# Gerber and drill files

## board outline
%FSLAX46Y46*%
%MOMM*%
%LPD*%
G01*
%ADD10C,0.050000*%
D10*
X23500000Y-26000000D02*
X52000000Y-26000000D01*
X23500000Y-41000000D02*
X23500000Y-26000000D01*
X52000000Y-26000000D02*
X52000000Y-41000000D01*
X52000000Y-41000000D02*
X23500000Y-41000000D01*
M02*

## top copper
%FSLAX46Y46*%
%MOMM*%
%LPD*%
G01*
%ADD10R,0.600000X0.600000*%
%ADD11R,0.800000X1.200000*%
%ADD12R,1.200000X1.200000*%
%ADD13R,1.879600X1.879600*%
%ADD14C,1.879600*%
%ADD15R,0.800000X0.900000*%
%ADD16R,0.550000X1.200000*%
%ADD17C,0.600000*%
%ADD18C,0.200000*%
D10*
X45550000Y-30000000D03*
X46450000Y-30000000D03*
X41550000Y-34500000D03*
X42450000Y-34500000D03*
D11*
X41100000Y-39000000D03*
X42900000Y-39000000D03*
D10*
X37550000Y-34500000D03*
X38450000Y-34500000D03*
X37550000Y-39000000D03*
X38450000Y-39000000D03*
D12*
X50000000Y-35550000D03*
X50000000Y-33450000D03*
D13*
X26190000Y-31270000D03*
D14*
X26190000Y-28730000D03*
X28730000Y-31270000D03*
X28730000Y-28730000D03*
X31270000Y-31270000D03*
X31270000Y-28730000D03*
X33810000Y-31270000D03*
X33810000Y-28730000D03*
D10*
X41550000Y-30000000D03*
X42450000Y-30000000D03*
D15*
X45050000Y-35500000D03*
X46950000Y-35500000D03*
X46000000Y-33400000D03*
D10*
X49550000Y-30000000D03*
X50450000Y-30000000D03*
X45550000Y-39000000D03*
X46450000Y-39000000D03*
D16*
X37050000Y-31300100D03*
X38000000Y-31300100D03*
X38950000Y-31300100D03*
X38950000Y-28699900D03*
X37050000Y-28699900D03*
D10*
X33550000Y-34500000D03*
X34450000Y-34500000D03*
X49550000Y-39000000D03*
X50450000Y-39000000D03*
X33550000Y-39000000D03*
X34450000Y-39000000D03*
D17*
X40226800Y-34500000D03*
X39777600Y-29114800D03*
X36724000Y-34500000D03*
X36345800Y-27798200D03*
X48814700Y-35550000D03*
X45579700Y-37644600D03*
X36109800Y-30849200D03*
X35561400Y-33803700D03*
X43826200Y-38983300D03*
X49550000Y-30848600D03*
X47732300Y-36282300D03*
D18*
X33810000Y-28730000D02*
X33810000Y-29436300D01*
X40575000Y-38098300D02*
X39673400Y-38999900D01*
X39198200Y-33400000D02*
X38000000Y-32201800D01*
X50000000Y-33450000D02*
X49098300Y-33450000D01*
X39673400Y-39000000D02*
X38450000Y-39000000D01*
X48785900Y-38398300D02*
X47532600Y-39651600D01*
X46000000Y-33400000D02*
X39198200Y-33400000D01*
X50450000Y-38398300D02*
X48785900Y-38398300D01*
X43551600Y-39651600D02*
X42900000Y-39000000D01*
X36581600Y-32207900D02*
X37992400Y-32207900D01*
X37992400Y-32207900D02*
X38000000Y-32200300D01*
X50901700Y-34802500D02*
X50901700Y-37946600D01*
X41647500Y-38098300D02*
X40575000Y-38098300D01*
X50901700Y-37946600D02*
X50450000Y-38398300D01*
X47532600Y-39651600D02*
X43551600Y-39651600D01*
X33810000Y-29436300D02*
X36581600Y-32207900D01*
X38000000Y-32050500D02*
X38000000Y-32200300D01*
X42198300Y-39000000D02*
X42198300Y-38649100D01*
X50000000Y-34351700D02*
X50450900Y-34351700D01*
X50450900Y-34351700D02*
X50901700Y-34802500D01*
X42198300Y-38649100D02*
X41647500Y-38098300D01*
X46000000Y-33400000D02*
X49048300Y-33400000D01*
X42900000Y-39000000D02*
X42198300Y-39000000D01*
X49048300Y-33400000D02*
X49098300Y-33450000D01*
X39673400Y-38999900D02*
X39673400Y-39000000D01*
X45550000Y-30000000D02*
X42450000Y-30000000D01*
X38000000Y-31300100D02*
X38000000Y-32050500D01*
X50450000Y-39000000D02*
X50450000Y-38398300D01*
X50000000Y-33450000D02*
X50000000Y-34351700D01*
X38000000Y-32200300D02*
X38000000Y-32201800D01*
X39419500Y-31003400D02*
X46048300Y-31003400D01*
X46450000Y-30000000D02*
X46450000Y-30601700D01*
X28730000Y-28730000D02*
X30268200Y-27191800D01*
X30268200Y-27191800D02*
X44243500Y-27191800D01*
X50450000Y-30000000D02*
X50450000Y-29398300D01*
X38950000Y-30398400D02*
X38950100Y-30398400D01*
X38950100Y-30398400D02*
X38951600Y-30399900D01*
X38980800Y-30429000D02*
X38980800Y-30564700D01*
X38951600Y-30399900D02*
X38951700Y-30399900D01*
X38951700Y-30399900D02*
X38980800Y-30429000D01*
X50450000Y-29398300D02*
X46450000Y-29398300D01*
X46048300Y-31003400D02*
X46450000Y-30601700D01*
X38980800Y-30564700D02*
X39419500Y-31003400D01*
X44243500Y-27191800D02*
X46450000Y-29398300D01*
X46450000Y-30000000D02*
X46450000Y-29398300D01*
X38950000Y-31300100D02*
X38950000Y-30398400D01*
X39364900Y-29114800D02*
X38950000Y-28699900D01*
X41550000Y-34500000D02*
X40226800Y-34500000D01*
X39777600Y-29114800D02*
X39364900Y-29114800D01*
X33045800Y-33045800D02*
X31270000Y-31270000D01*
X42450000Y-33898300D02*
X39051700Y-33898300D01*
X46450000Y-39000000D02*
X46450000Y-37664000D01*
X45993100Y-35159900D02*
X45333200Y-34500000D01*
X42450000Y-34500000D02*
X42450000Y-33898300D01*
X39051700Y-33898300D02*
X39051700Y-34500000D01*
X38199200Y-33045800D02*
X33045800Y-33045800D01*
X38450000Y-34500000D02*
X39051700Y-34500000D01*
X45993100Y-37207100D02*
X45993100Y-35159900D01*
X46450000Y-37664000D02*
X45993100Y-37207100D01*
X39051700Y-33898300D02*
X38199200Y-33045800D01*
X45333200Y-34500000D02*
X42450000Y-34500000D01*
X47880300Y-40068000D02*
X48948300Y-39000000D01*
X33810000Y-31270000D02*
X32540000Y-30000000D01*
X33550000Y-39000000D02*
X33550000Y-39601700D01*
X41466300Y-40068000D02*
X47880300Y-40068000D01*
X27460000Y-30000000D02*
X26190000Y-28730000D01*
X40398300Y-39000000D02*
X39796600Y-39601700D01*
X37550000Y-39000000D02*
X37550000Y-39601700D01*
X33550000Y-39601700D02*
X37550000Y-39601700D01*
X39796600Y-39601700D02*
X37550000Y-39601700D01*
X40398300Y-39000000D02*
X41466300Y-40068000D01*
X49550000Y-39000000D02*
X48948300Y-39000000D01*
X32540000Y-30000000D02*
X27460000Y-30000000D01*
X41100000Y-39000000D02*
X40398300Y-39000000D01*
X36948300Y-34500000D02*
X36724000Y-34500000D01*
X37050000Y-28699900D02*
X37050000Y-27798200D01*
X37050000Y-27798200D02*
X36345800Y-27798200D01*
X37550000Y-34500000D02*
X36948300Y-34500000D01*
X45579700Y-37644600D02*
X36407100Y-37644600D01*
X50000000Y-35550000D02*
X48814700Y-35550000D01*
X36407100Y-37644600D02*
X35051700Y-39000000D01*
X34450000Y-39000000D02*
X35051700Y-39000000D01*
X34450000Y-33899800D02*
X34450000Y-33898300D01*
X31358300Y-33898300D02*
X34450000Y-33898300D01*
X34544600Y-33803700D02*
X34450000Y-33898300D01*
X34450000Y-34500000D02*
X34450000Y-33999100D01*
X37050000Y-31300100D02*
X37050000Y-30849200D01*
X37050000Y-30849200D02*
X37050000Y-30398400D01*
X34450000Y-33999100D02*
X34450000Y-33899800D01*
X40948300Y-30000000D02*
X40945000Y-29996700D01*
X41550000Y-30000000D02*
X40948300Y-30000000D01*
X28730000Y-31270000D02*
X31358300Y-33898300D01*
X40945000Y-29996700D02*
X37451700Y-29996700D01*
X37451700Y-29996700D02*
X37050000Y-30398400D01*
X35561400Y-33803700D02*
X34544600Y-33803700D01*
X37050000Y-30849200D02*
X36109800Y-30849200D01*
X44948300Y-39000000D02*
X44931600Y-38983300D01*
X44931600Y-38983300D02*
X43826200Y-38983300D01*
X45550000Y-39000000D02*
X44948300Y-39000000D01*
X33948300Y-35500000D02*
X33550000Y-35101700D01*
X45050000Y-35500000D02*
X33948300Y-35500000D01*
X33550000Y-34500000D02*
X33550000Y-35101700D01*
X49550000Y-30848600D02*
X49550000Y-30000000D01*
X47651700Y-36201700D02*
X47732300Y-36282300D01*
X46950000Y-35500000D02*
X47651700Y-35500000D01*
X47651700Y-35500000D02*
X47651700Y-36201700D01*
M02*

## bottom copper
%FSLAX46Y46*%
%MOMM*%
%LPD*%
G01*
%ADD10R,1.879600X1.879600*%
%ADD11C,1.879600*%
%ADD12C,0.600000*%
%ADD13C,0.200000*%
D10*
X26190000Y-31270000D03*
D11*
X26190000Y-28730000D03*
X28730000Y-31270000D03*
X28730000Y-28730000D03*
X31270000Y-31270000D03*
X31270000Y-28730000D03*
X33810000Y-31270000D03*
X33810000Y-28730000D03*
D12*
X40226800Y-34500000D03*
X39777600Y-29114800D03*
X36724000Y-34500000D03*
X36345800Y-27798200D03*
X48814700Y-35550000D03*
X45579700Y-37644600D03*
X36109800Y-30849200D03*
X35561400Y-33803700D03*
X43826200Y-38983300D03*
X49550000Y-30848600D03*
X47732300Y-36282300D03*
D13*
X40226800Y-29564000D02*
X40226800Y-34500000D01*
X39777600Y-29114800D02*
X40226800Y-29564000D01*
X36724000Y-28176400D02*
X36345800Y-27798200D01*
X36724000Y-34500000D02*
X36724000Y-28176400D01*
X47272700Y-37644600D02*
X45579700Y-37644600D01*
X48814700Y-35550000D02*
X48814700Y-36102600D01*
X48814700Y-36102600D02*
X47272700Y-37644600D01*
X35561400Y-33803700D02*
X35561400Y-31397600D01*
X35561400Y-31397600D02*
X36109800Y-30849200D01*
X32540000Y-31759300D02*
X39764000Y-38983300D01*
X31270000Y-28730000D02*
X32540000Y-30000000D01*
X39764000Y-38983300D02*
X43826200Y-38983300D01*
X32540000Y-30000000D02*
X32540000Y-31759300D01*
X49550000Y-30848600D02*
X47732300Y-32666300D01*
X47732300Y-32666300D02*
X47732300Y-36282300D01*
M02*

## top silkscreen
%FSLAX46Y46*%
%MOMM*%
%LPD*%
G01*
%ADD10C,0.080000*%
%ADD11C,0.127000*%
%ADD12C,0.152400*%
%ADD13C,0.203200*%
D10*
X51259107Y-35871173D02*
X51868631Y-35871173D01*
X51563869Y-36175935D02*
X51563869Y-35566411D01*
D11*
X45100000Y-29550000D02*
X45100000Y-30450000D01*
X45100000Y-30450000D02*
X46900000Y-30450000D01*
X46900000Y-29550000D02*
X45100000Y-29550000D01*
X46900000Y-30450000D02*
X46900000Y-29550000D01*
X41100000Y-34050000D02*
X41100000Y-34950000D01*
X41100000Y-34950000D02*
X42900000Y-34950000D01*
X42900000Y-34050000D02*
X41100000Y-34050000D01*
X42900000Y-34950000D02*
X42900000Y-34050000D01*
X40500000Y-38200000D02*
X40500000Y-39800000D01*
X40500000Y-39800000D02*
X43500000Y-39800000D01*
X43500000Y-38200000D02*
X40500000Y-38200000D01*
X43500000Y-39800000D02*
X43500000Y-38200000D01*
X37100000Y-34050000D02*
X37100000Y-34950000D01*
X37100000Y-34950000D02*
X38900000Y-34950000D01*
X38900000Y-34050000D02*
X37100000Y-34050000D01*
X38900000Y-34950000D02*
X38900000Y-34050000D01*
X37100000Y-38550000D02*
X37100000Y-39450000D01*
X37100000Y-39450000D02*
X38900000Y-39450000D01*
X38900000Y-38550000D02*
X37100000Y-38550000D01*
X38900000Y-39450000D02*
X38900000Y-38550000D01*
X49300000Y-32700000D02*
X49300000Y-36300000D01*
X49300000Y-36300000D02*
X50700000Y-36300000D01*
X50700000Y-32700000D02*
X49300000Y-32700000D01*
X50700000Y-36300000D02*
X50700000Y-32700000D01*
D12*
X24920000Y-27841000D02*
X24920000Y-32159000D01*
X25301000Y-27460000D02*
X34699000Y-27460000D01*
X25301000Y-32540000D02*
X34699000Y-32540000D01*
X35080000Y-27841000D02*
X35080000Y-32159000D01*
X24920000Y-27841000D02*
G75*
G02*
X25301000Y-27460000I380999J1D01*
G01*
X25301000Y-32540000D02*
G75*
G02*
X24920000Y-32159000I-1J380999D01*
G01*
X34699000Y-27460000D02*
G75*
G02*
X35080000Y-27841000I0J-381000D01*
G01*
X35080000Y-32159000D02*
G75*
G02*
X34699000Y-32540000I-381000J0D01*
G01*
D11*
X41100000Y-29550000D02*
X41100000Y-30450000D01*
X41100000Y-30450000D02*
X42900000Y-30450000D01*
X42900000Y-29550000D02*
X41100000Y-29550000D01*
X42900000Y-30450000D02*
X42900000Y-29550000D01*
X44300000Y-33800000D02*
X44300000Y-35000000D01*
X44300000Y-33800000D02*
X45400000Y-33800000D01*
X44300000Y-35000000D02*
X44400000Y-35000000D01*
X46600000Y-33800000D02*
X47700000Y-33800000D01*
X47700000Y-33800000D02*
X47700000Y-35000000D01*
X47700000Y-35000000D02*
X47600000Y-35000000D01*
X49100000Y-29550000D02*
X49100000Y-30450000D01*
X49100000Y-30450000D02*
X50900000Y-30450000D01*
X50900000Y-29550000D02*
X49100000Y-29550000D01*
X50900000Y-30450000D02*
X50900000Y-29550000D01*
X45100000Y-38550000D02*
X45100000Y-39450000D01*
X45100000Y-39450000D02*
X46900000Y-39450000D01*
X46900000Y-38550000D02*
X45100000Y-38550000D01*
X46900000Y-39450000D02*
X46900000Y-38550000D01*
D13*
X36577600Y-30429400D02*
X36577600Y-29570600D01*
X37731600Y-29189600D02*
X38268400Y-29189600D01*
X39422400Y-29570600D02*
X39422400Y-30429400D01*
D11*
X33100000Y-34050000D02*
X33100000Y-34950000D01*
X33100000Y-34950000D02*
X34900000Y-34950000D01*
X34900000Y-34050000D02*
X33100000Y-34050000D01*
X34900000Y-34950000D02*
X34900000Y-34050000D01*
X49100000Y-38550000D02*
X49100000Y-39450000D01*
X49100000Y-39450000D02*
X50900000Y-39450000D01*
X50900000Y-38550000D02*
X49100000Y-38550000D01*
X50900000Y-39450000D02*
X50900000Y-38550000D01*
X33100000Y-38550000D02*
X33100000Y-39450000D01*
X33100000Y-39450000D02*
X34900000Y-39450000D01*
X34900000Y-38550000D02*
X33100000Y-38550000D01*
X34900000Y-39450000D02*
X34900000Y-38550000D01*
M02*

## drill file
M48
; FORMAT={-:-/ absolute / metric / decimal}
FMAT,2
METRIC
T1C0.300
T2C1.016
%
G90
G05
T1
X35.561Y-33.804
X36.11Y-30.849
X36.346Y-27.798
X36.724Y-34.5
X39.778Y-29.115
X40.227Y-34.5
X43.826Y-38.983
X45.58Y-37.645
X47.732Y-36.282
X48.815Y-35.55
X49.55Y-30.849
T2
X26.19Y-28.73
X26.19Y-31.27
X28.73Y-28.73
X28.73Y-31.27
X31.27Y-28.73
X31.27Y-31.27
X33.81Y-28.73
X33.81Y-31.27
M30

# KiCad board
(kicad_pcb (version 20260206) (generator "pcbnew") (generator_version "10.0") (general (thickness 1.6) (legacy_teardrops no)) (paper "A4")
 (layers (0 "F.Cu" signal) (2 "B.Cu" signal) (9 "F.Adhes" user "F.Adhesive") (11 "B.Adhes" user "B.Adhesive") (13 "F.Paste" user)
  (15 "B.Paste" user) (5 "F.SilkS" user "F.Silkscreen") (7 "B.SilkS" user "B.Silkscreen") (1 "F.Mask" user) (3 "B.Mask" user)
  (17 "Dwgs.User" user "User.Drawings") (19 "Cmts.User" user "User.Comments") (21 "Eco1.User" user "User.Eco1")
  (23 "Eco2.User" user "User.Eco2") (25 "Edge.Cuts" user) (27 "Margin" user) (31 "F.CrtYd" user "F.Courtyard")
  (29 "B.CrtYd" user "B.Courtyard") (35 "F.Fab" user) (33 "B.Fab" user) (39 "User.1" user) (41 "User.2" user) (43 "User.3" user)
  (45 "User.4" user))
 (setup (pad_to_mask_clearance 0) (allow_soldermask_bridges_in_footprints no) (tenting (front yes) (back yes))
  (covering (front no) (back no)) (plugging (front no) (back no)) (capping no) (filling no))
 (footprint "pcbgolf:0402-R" (layer "F.Cu") (at 46 30)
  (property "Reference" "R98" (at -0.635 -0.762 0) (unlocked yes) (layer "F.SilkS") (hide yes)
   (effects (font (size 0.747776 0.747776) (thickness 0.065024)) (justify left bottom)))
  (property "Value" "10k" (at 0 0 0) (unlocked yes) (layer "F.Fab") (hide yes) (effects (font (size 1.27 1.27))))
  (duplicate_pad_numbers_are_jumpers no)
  (fp_line (start -0.9 -0.45) (end -0.9 0.45) (stroke (width 0.127) (type solid)) (layer "F.SilkS"))
  (fp_line (start -0.9 0.45) (end 0.9 0.45) (stroke (width 0.127) (type solid)) (layer "F.SilkS"))
  (fp_line (start 0.9 -0.45) (end -0.9 -0.45) (stroke (width 0.127) (type solid)) (layer "F.SilkS"))
  (fp_line (start 0.9 0.45) (end 0.9 -0.45) (stroke (width 0.127) (type solid)) (layer "F.SilkS"))
  (pad "1" smd rect (at -0.45 0) (size 0.6 0.6) (layers "F.Cu" "F.Mask" "F.Paste") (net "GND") (solder_mask_margin 0.0508)
   (solder_paste_margin 0) (thermal_bridge_angle 0))
  (pad "2" smd rect (at 0.45 0) (size 0.6 0.6) (layers "F.Cu" "F.Mask" "F.Paste") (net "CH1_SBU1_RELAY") (solder_mask_margin 0.0508)
   (solder_paste_margin 0) (thermal_bridge_angle 0)))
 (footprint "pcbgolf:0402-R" (layer "F.Cu") (at 42 34.5)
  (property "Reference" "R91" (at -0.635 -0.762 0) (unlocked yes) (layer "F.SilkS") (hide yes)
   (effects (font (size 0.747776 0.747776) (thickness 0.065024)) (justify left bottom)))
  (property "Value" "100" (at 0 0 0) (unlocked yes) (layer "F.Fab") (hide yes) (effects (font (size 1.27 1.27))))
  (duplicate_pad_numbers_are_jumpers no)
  (fp_line (start -0.9 -0.45) (end -0.9 0.45) (stroke (width 0.127) (type solid)) (layer "F.SilkS"))
  (fp_line (start -0.9 0.45) (end 0.9 0.45) (stroke (width 0.127) (type solid)) (layer "F.SilkS"))
  (fp_line (start 0.9 -0.45) (end -0.9 -0.45) (stroke (width 0.127) (type solid)) (layer "F.SilkS"))
  (fp_line (start 0.9 0.45) (end 0.9 -0.45) (stroke (width 0.127) (type solid)) (layer "F.SilkS"))
  (pad "1" smd rect (at -0.45 0) (size 0.6 0.6) (layers "F.Cu" "F.Mask" "F.Paste") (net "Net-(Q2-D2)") (solder_mask_margin 0.0508)
   (solder_paste_margin 0) (thermal_bridge_angle 0))
  (pad "2" smd rect (at 0.45 0) (size 0.6 0.6) (layers "F.Cu" "F.Mask" "F.Paste") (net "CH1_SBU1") (solder_mask_margin 0.0508)
   (solder_paste_margin 0) (thermal_bridge_angle 0)))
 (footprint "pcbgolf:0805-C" (layer "F.Cu") (at 42 39)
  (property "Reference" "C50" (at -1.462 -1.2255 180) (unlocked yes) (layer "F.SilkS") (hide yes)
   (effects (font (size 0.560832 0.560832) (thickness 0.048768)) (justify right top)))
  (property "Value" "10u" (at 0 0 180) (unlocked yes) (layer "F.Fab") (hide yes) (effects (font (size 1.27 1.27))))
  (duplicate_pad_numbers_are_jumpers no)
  (fp_line (start -1.5 -0.8) (end -1.5 0.8) (stroke (width 0.127) (type solid)) (layer "F.SilkS"))
  (fp_line (start -1.5 0.8) (end 1.5 0.8) (stroke (width 0.127) (type solid)) (layer "F.SilkS"))
  (fp_line (start 1.5 -0.8) (end -1.5 -0.8) (stroke (width 0.127) (type solid)) (layer "F.SilkS"))
  (fp_line (start 1.5 0.8) (end 1.5 -0.8) (stroke (width 0.127) (type solid)) (layer "F.SilkS"))
  (pad "1" smd rect (at -0.9 0) (size 0.8 1.2) (layers "F.Cu" "F.Mask" "F.Paste") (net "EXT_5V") (solder_mask_margin 0.0508)
   (solder_paste_margin 0) (thermal_bridge_angle 0))
  (pad "2" smd rect (at 0.9 0) (size 0.8 1.2) (layers "F.Cu" "F.Mask" "F.Paste") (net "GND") (solder_mask_margin 0.0508)
   (solder_paste_margin 0) (thermal_bridge_angle 0)))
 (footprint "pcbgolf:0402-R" (layer "F.Cu") (at 38 34.5)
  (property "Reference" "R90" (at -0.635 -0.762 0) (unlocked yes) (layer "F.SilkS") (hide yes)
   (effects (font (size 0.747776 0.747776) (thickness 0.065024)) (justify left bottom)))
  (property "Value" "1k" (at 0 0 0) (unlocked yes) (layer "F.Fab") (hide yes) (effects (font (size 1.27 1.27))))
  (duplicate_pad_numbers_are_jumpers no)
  (fp_line (start -0.9 -0.45) (end -0.9 0.45) (stroke (width 0.127) (type solid)) (layer "F.SilkS"))
  (fp_line (start -0.9 0.45) (end 0.9 0.45) (stroke (width 0.127) (type solid)) (layer "F.SilkS"))
  (fp_line (start 0.9 -0.45) (end -0.9 -0.45) (stroke (width 0.127) (type solid)) (layer "F.SilkS"))
  (fp_line (start 0.9 0.45) (end 0.9 -0.45) (stroke (width 0.127) (type solid)) (layer "F.SilkS"))
  (pad "1" smd rect (at -0.45 0) (size 0.6 0.6) (layers "F.Cu" "F.Mask" "F.Paste") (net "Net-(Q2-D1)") (solder_mask_margin 0.0508)
   (solder_paste_margin 0) (thermal_bridge_angle 0))
  (pad "2" smd rect (at 0.45 0) (size 0.6 0.6) (layers "F.Cu" "F.Mask" "F.Paste") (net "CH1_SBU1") (solder_mask_margin 0.0508)
   (solder_paste_margin 0) (thermal_bridge_angle 0)))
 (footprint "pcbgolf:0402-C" (layer "F.Cu") (at 38 39)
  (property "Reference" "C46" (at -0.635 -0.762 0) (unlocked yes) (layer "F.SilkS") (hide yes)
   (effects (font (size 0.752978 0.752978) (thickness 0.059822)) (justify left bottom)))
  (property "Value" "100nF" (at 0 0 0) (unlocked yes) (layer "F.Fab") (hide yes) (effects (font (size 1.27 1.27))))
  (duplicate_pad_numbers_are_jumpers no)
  (fp_line (start -0.9 -0.45) (end -0.9 0.45) (stroke (width 0.127) (type solid)) (layer "F.SilkS"))
  (fp_line (start -0.9 0.45) (end 0.9 0.45) (stroke (width 0.127) (type solid)) (layer "F.SilkS"))
  (fp_line (start 0.9 -0.45) (end -0.9 -0.45) (stroke (width 0.127) (type solid)) (layer "F.SilkS"))
  (fp_line (start 0.9 0.45) (end 0.9 -0.45) (stroke (width 0.127) (type solid)) (layer "F.SilkS"))
  (pad "1" smd rect (at -0.45 0) (size 0.6 0.6) (layers "F.Cu" "F.Mask" "F.Paste") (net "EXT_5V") (solder_mask_margin 0.0508)
   (solder_paste_margin 0) (thermal_bridge_angle 0))
  (pad "2" smd rect (at 0.45 0) (size 0.6 0.6) (layers "F.Cu" "F.Mask" "F.Paste") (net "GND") (solder_mask_margin 0.0508)
   (solder_paste_margin 0) (thermal_bridge_angle 0)))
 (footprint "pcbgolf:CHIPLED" (layer "F.Cu") (at 50 34.5)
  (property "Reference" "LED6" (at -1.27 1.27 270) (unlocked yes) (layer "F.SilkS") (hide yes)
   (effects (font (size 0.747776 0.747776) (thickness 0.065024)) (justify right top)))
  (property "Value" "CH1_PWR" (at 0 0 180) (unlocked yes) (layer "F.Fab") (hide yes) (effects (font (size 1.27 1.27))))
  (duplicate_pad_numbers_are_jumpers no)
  (fp_line (start -0.7 -1.8) (end -0.7 1.8) (stroke (width 0.127) (type solid)) (layer "F.SilkS"))
  (fp_line (start -0.7 1.8) (end 0.7 1.8) (stroke (width 0.127) (type solid)) (layer "F.SilkS"))
  (fp_line (start 0.7 -1.8) (end -0.7 -1.8) (stroke (width 0.127) (type solid)) (layer "F.SilkS"))
  (fp_line (start 0.7 1.8) (end 0.7 -1.8) (stroke (width 0.127) (type solid)) (layer "F.SilkS"))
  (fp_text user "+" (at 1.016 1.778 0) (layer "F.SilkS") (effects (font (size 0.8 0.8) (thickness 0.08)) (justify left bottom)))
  (pad "A" smd rect (at 0 1.05) (size 1.2 1.2) (layers "F.Cu" "F.Mask" "F.Paste") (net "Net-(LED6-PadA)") (solder_mask_margin 0.0508)
   (solder_paste_margin 0) (thermal_bridge_angle 0))
  (pad "C" smd rect (at 0 -1.05) (size 1.2 1.2) (layers "F.Cu" "F.Mask" "F.Paste") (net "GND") (solder_mask_margin 0.0508)
   (solder_paste_margin 0) (thermal_bridge_angle 0)))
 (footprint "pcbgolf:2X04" (layer "F.Cu") (at 30 30)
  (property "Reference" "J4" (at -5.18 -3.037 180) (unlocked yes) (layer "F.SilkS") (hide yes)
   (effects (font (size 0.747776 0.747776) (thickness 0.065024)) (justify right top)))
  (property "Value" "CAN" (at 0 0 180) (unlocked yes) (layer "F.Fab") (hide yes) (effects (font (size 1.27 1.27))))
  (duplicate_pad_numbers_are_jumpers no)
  (fp_line (start -5.08 -2.159) (end -5.08 2.159) (stroke (width 0.1524) (type solid)) (layer "F.SilkS"))
  (fp_line (start -4.699 -2.54) (end 4.699 -2.54) (stroke (width 0.1524) (type solid)) (layer "F.SilkS"))
  (fp_line (start -4.699 2.54) (end 4.699 2.54) (stroke (width 0.1524) (type solid)) (layer "F.SilkS"))
  (fp_line (start 5.08 -2.159) (end 5.08 2.159) (stroke (width 0.1524) (type solid)) (layer "F.SilkS"))
  (fp_arc (start -5.08 -2.159) (mid -4.968408 -2.428408) (end -4.699 -2.54) (stroke (width 0.1524) (type solid)) (layer "F.SilkS"))
  (fp_arc (start -4.699 2.54) (mid -4.968408 2.428408) (end -5.08 2.159) (stroke (width 0.1524) (type solid)) (layer "F.SilkS"))
  (fp_arc (start 4.699 -2.54) (mid 4.968408 -2.428408) (end 5.08 -2.159) (stroke (width 0.1524) (type solid)) (layer "F.SilkS"))
  (fp_arc (start 5.08 2.159) (mid 4.968408 2.428408) (end 4.699 2.54) (stroke (width 0.1524) (type solid)) (layer "F.SilkS"))
  (pad "1" thru_hole rect (at -3.81 1.27 90) (size 1.8796 1.8796) (drill 1.016) (layers "*.Cu" "*.Mask") (remove_unused_layers no)
   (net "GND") (solder_mask_margin 0.0508) (thermal_bridge_angle 0))
  (pad "2" thru_hole circle (at -3.81 -1.27 90) (size 1.8796 1.8796) (drill 1.016) (layers "*.Cu" "*.Mask") (remove_unused_layers no)
   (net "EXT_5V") (solder_mask_margin 0.0508) (thermal_bridge_angle 0))
  (pad "3" thru_hole circle (at -1.27 1.27 90) (size 1.8796 1.8796) (drill 1.016) (layers "*.Cu" "*.Mask") (remove_unused_layers no)
   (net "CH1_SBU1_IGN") (solder_mask_margin 0.0508) (thermal_bridge_angle 0))
  (pad "4" thru_hole circle (at -1.27 -1.27 90) (size 1.8796 1.8796) (drill 1.016) (layers "*.Cu" "*.Mask") (remove_unused_layers no)
   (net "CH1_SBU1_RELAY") (solder_mask_margin 0.0508) (thermal_bridge_angle 0))
  (pad "5" thru_hole circle (at 1.27 1.27 90) (size 1.8796 1.8796) (drill 1.016) (layers "*.Cu" "*.Mask") (remove_unused_layers no)
   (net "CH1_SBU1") (solder_mask_margin 0.0508) (thermal_bridge_angle 0))
  (pad "6" thru_hole circle (at 1.27 -1.27 90) (size 1.8796 1.8796) (drill 1.016) (layers "*.Cu" "*.Mask") (remove_unused_layers no)
   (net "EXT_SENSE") (solder_mask_margin 0.0508) (thermal_bridge_angle 0))
  (pad "7" thru_hole circle (at 3.81 1.27 90) (size 1.8796 1.8796) (drill 1.016) (layers "*.Cu" "*.Mask") (remove_unused_layers no)
   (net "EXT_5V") (solder_mask_margin 0.0508) (thermal_bridge_angle 0))
  (pad "8" thru_hole circle (at 3.81 -1.27 90) (size 1.8796 1.8796) (drill 1.016) (layers "*.Cu" "*.Mask") (remove_unused_layers no)
   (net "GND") (solder_mask_margin 0.0508) (thermal_bridge_angle 0)))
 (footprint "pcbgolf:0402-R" (layer "F.Cu") (at 42 30)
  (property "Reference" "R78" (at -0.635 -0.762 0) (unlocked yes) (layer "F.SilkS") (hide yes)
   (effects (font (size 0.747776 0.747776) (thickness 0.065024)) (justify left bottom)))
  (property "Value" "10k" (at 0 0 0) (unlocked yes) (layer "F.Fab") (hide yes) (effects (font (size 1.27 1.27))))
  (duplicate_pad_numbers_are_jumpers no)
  (fp_line (start -0.9 -0.45) (end -0.9 0.45) (stroke (width 0.127) (type solid)) (layer "F.SilkS"))
  (fp_line (start -0.9 0.45) (end 0.9 0.45) (stroke (width 0.127) (type solid)) (layer "F.SilkS"))
  (fp_line (start 0.9 -0.45) (end -0.9 -0.45) (stroke (width 0.127) (type solid)) (layer "F.SilkS"))
  (fp_line (start 0.9 0.45) (end 0.9 -0.45) (stroke (width 0.127) (type solid)) (layer "F.SilkS"))
  (pad "1" smd rect (at -0.45 0) (size 0.6 0.6) (layers "F.Cu" "F.Mask" "F.Paste") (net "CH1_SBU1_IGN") (solder_mask_margin 0.0508)
   (solder_paste_margin 0) (thermal_bridge_angle 0))
  (pad "2" smd rect (at 0.45 0) (size 0.6 0.6) (layers "F.Cu" "F.Mask" "F.Paste") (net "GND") (solder_mask_margin 0.0508)
   (solder_paste_margin 0) (thermal_bridge_angle 0)))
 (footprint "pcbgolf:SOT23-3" (layer "F.Cu") (at 46 34.5)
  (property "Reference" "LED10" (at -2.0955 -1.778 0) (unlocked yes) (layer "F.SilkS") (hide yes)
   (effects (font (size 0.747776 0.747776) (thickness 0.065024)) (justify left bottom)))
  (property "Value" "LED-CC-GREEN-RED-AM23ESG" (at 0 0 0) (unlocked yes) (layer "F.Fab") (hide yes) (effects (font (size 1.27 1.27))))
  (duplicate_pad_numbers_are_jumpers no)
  (fp_line (start -1.7 -0.7) (end -1.7 0.5) (stroke (width 0.127) (type solid)) (layer "F.SilkS"))
  (fp_line (start -1.7 -0.7) (end -0.6 -0.7) (stroke (width 0.127) (type solid)) (layer "F.SilkS"))
  (fp_line (start -1.7 0.5) (end -1.6 0.5) (stroke (width 0.127) (type solid)) (layer "F.SilkS"))
  (fp_line (start 0.6 -0.7) (end 1.7 -0.7) (stroke (width 0.127) (type solid)) (layer "F.SilkS"))
  (fp_line (start 1.7 -0.7) (end 1.7 0.5) (stroke (width 0.127) (type solid)) (layer "F.SilkS"))
  (fp_line (start 1.7 0.5) (end 1.6 0.5) (stroke (width 0.127) (type solid)) (layer "F.SilkS"))
  (pad "1" smd rect (at -0.95 1) (size 0.8 0.9) (layers "F.Cu" "F.Mask" "F.Paste") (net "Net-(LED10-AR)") (solder_mask_margin 0.0508)
   (solder_paste_margin 0) (thermal_bridge_angle 0))
  (pad "2" smd rect (at 0.95 1) (size 0.8 0.9) (layers "F.Cu" "F.Mask" "F.Paste") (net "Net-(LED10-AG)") (solder_mask_margin 0.0508)
   (solder_paste_margin 0) (thermal_bridge_angle 0))
  (pad "3" smd rect (at 0 -1.1) (size 0.8 0.9) (layers "F.Cu" "F.Mask" "F.Paste") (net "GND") (solder_mask_margin 0.0508)
   (solder_paste_margin 0) (thermal_bridge_angle 0)))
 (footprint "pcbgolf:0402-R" (layer "F.Cu") (at 50 30)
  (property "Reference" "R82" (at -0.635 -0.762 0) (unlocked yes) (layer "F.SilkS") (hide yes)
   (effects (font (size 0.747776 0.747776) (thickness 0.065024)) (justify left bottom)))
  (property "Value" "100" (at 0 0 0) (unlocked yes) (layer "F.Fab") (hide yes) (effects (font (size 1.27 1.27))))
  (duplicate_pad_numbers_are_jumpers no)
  (fp_line (start -0.9 -0.45) (end -0.9 0.45) (stroke (width 0.127) (type solid)) (layer "F.SilkS"))
  (fp_line (start -0.9 0.45) (end 0.9 0.45) (stroke (width 0.127) (type solid)) (layer "F.SilkS"))
  (fp_line (start 0.9 -0.45) (end -0.9 -0.45) (stroke (width 0.127) (type solid)) (layer "F.SilkS"))
  (fp_line (start 0.9 0.45) (end 0.9 -0.45) (stroke (width 0.127) (type solid)) (layer "F.SilkS"))
  (pad "1" smd rect (at -0.45 0) (size 0.6 0.6) (layers "F.Cu" "F.Mask" "F.Paste") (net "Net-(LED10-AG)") (solder_mask_margin 0.0508)
   (solder_paste_margin 0) (thermal_bridge_angle 0))
  (pad "2" smd rect (at 0.45 0) (size 0.6 0.6) (layers "F.Cu" "F.Mask" "F.Paste") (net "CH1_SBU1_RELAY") (solder_mask_margin 0.0508)
   (solder_paste_margin 0) (thermal_bridge_angle 0)))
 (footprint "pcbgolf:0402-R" (layer "F.Cu") (at 46 39)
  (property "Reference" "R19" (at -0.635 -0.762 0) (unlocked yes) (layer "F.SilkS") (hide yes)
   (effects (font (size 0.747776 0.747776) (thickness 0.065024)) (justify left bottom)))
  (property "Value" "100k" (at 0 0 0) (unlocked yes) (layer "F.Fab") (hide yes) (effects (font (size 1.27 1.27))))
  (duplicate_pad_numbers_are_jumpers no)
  (fp_line (start -0.9 -0.45) (end -0.9 0.45) (stroke (width 0.127) (type solid)) (layer "F.SilkS"))
  (fp_line (start -0.9 0.45) (end 0.9 0.45) (stroke (width 0.127) (type solid)) (layer "F.SilkS"))
  (fp_line (start 0.9 -0.45) (end -0.9 -0.45) (stroke (width 0.127) (type solid)) (layer "F.SilkS"))
  (fp_line (start 0.9 0.45) (end 0.9 -0.45) (stroke (width 0.127) (type solid)) (layer "F.SilkS"))
  (pad "1" smd rect (at -0.45 0) (size 0.6 0.6) (layers "F.Cu" "F.Mask" "F.Paste") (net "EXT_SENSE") (solder_mask_margin 0.0508)
   (solder_paste_margin 0) (thermal_bridge_angle 0))
  (pad "2" smd rect (at 0.45 0) (size 0.6 0.6) (layers "F.Cu" "F.Mask" "F.Paste") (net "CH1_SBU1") (solder_mask_margin 0.0508)
   (solder_paste_margin 0) (thermal_bridge_angle 0)))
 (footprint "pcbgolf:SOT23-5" (layer "F.Cu") (at 38 30)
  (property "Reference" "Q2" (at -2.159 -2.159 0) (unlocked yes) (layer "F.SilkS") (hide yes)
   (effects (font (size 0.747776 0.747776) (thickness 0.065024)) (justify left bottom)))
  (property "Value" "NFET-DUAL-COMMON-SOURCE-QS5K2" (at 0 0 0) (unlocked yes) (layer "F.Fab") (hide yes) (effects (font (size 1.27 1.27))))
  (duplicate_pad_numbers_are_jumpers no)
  (fp_line (start -1.4224 0.4294) (end -1.4224 -0.4294) (stroke (width 0.2032) (type solid)) (layer "F.SilkS"))
  (fp_line (start -0.2684 -0.8104) (end 0.2684 -0.8104) (stroke (width 0.2032) (type solid)) (layer "F.SilkS"))
  (fp_line (start 1.4224 -0.4294) (end 1.4224 0.4294) (stroke (width 0.2032) (type solid)) (layer "F.SilkS"))
  (pad "1" smd rect (at -0.95 1.3001) (size 0.55 1.2) (layers "F.Cu" "F.Mask" "F.Paste") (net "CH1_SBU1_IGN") (solder_mask_margin 0.0508)
   (solder_paste_margin 0) (thermal_bridge_angle 0))
  (pad "2" smd rect (at 0 1.3001) (size 0.55 1.2) (layers "F.Cu" "F.Mask" "F.Paste") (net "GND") (solder_mask_margin 0.0508)
   (solder_paste_margin 0) (thermal_bridge_angle 0))
  (pad "3" smd rect (at 0.95 1.3001) (size 0.55 1.2) (layers "F.Cu" "F.Mask" "F.Paste") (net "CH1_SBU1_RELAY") (solder_mask_margin 0.0508)
   (solder_paste_margin 0) (thermal_bridge_angle 0))
  (pad "4" smd rect (at 0.95 -1.3001) (size 0.55 1.2) (layers "F.Cu" "F.Mask" "F.Paste") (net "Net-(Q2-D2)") (solder_mask_margin 0.0508)
   (solder_paste_margin 0) (thermal_bridge_angle 0))
  (pad "5" smd rect (at -0.95 -1.3001) (size 0.55 1.2) (layers "F.Cu" "F.Mask" "F.Paste") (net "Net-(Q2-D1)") (solder_mask_margin 0.0508)
   (solder_paste_margin 0) (thermal_bridge_angle 0)))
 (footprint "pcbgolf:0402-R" (layer "F.Cu") (at 34 34.5)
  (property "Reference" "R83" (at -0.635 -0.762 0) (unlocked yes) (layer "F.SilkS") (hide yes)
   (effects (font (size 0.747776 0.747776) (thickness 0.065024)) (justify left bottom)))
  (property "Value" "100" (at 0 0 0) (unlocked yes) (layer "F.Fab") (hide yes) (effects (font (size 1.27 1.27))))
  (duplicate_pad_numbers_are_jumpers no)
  (fp_line (start -0.9 -0.45) (end -0.9 0.45) (stroke (width 0.127) (type solid)) (layer "F.SilkS"))
  (fp_line (start -0.9 0.45) (end 0.9 0.45) (stroke (width 0.127) (type solid)) (layer "F.SilkS"))
  (fp_line (start 0.9 -0.45) (end -0.9 -0.45) (stroke (width 0.127) (type solid)) (layer "F.SilkS"))
  (fp_line (start 0.9 0.45) (end 0.9 -0.45) (stroke (width 0.127) (type solid)) (layer "F.SilkS"))
  (pad "1" smd rect (at -0.45 0) (size 0.6 0.6) (layers "F.Cu" "F.Mask" "F.Paste") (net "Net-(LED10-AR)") (solder_mask_margin 0.0508)
   (solder_paste_margin 0) (thermal_bridge_angle 0))
  (pad "2" smd rect (at 0.45 0) (size 0.6 0.6) (layers "F.Cu" "F.Mask" "F.Paste") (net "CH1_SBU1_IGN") (solder_mask_margin 0.0508)
   (solder_paste_margin 0) (thermal_bridge_angle 0)))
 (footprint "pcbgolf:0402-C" (layer "F.Cu") (at 50 39)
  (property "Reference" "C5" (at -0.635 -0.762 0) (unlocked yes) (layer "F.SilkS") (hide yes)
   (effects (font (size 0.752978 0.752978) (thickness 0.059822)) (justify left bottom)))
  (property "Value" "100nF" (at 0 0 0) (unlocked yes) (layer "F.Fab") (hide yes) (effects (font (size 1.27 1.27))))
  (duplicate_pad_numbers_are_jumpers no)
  (fp_line (start -0.9 -0.45) (end -0.9 0.45) (stroke (width 0.127) (type solid)) (layer "F.SilkS"))
  (fp_line (start -0.9 0.45) (end 0.9 0.45) (stroke (width 0.127) (type solid)) (layer "F.SilkS"))
  (fp_line (start 0.9 -0.45) (end -0.9 -0.45) (stroke (width 0.127) (type solid)) (layer "F.SilkS"))
  (fp_line (start 0.9 0.45) (end 0.9 -0.45) (stroke (width 0.127) (type solid)) (layer "F.SilkS"))
  (pad "1" smd rect (at -0.45 0) (size 0.6 0.6) (layers "F.Cu" "F.Mask" "F.Paste") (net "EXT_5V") (solder_mask_margin 0.0508)
   (solder_paste_margin 0) (thermal_bridge_angle 0))
  (pad "2" smd rect (at 0.45 0) (size 0.6 0.6) (layers "F.Cu" "F.Mask" "F.Paste") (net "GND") (solder_mask_margin 0.0508)
   (solder_paste_margin 0) (thermal_bridge_angle 0)))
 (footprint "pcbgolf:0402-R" (layer "F.Cu") (at 34 39)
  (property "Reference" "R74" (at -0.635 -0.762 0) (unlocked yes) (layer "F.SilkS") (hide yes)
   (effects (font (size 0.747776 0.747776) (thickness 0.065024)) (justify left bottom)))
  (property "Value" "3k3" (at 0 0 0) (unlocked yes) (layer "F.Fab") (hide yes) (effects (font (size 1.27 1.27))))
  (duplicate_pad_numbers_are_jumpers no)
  (fp_line (start -0.9 -0.45) (end -0.9 0.45) (stroke (width 0.127) (type solid)) (layer "F.SilkS"))
  (fp_line (start -0.9 0.45) (end 0.9 0.45) (stroke (width 0.127) (type solid)) (layer "F.SilkS"))
  (fp_line (start 0.9 -0.45) (end -0.9 -0.45) (stroke (width 0.127) (type solid)) (layer "F.SilkS"))
  (fp_line (start 0.9 0.45) (end 0.9 -0.45) (stroke (width 0.127) (type solid)) (layer "F.SilkS"))
  (pad "1" smd rect (at -0.45 0) (size 0.6 0.6) (layers "F.Cu" "F.Mask" "F.Paste") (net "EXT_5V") (solder_mask_margin 0.0508)
   (solder_paste_margin 0) (thermal_bridge_angle 0))
  (pad "2" smd rect (at 0.45 0) (size 0.6 0.6) (layers "F.Cu" "F.Mask" "F.Paste") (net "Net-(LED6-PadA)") (solder_mask_margin 0.0508)
   (solder_paste_margin 0) (thermal_bridge_angle 0)))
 (gr_line (start 23.5 26) (end 52 26) (stroke (width 0.05) (type default)) (layer "Edge.Cuts"))
 (gr_line (start 23.5 41) (end 23.5 26) (stroke (width 0.05) (type default)) (layer "Edge.Cuts"))
 (gr_line (start 52 26) (end 52 41) (stroke (width 0.05) (type default)) (layer "Edge.Cuts"))
 (gr_line (start 52 41) (end 23.5 41) (stroke (width 0.05) (type default)) (layer "Edge.Cuts"))
 (segment (start 33.81 28.73) (end 33.81 29.4363) (width 0.2) (layer "F.Cu") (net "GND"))
 (segment (start 40.575 38.0983) (end 39.6734 38.9999) (width 0.2) (layer "F.Cu") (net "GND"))
 (segment (start 39.1982 33.4) (end 38 32.2018) (width 0.2) (layer "F.Cu") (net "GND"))
 (segment (start 50 33.45) (end 49.0983 33.45) (width 0.2) (layer "F.Cu") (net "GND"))
 (segment (start 39.6734 39) (end 38.45 39) (width 0.2) (layer "F.Cu") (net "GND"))
 (segment (start 48.7859 38.3983) (end 47.5326 39.6516) (width 0.2) (layer "F.Cu") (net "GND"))
 (segment (start 46 33.4) (end 39.1982 33.4) (width 0.2) (layer "F.Cu") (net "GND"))
 (segment (start 50.45 38.3983) (end 48.7859 38.3983) (width 0.2) (layer "F.Cu") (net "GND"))
 (segment (start 43.5516 39.6516) (end 42.9 39) (width 0.2) (layer "F.Cu") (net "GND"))
 (segment (start 36.5816 32.2079) (end 37.9924 32.2079) (width 0.2) (layer "F.Cu") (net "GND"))
 (segment (start 37.9924 32.2079) (end 38 32.2003) (width 0.2) (layer "F.Cu") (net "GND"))
 (segment (start 50.9017 34.8025) (end 50.9017 37.9466) (width 0.2) (layer "F.Cu") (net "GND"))
 (segment (start 41.6475 38.0983) (end 40.575 38.0983) (width 0.2) (layer "F.Cu") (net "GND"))
 (segment (start 50.9017 37.9466) (end 50.45 38.3983) (width 0.2) (layer "F.Cu") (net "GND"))
 (segment (start 47.5326 39.6516) (end 43.5516 39.6516) (width 0.2) (layer "F.Cu") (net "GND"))
 (segment (start 33.81 29.4363) (end 36.5816 32.2079) (width 0.2) (layer "F.Cu") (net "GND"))
 (segment (start 38 32.0505) (end 38 32.2003) (width 0.2) (layer "F.Cu") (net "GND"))
 (segment (start 42.1983 39) (end 42.1983 38.6491) (width 0.2) (layer "F.Cu") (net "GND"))
 (segment (start 50 34.3517) (end 50.4509 34.3517) (width 0.2) (layer "F.Cu") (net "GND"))
 (segment (start 50.4509 34.3517) (end 50.9017 34.8025) (width 0.2) (layer "F.Cu") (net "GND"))
 (segment (start 42.1983 38.6491) (end 41.6475 38.0983) (width 0.2) (layer "F.Cu") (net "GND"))
 (segment (start 46 33.4) (end 49.0483 33.4) (width 0.2) (layer "F.Cu") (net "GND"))
 (segment (start 42.9 39) (end 42.1983 39) (width 0.2) (layer "F.Cu") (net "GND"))
 (segment (start 49.0483 33.4) (end 49.0983 33.45) (width 0.2) (layer "F.Cu") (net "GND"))
 (segment (start 39.6734 38.9999) (end 39.6734 39) (width 0.2) (layer "F.Cu") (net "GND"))
 (segment (start 45.55 30) (end 42.45 30) (width 0.2) (layer "F.Cu") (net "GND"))
 (segment (start 38 31.3001) (end 38 32.0505) (width 0.2) (layer "F.Cu") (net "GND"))
 (segment (start 50.45 39) (end 50.45 38.3983) (width 0.2) (layer "F.Cu") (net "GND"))
 (segment (start 50 33.45) (end 50 34.3517) (width 0.2) (layer "F.Cu") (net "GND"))
 (segment (start 38 32.2003) (end 38 32.2018) (width 0.2) (layer "F.Cu") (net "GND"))
 (segment (start 39.4195 31.0034) (end 46.0483 31.0034) (width 0.2) (layer "F.Cu") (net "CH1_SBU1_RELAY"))
 (segment (start 46.45 30) (end 46.45 30.6017) (width 0.2) (layer "F.Cu") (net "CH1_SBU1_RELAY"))
 (segment (start 28.73 28.73) (end 30.2682 27.1918) (width 0.2) (layer "F.Cu") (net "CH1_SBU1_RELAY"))
 (segment (start 30.2682 27.1918) (end 44.2435 27.1918) (width 0.2) (layer "F.Cu") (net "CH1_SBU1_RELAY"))
 (segment (start 50.45 30) (end 50.45 29.3983) (width 0.2) (layer "F.Cu") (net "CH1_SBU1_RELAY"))
 (segment (start 38.95 30.3984) (end 38.9501 30.3984) (width 0.2) (layer "F.Cu") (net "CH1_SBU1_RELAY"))
 (segment (start 38.9501 30.3984) (end 38.9516 30.3999) (width 0.2) (layer "F.Cu") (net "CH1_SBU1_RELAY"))
 (segment (start 38.9808 30.429) (end 38.9808 30.5647) (width 0.2) (layer "F.Cu") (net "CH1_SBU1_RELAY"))
 (segment (start 38.9516 30.3999) (end 38.9517 30.3999) (width 0.2) (layer "F.Cu") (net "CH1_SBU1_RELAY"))
 (segment (start 38.9517 30.3999) (end 38.9808 30.429) (width 0.2) (layer "F.Cu") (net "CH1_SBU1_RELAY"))
 (segment (start 50.45 29.3983) (end 46.45 29.3983) (width 0.2) (layer "F.Cu") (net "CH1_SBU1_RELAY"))
 (segment (start 46.0483 31.0034) (end 46.45 30.6017) (width 0.2) (layer "F.Cu") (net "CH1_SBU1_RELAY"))
 (segment (start 38.9808 30.5647) (end 39.4195 31.0034) (width 0.2) (layer "F.Cu") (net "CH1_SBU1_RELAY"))
 (segment (start 44.2435 27.1918) (end 46.45 29.3983) (width 0.2) (layer "F.Cu") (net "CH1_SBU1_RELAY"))
 (segment (start 46.45 30) (end 46.45 29.3983) (width 0.2) (layer "F.Cu") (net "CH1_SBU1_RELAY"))
 (segment (start 38.95 31.3001) (end 38.95 30.3984) (width 0.2) (layer "F.Cu") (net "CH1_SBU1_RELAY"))
 (segment (start 39.3649 29.1148) (end 38.95 28.6999) (width 0.2) (layer "F.Cu") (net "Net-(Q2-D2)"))
 (segment (start 41.55 34.5) (end 40.2268 34.5) (width 0.2) (layer "F.Cu") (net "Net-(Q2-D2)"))
 (segment (start 39.7776 29.1148) (end 39.3649 29.1148) (width 0.2) (layer "F.Cu") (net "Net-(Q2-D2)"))
 (via (at 40.2268 34.5) (size 0.6) (drill 0.3) (layers "F.Cu" "B.Cu") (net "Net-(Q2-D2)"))
 (via (at 39.7776 29.1148) (size 0.6) (drill 0.3) (layers "F.Cu" "B.Cu") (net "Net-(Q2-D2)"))
 (segment (start 40.2268 29.564) (end 40.2268 34.5) (width 0.2) (layer "B.Cu") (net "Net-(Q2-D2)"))
 (segment (start 39.7776 29.1148) (end 40.2268 29.564) (width 0.2) (layer "B.Cu") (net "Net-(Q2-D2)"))
 (segment (start 33.0458 33.0458) (end 31.27 31.27) (width 0.2) (layer "F.Cu") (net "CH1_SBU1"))
 (segment (start 42.45 33.8983) (end 39.0517 33.8983) (width 0.2) (layer "F.Cu") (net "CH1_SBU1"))
 (segment (start 46.45 39) (end 46.45 37.664) (width 0.2) (layer "F.Cu") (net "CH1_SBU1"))
 (segment (start 45.9931 35.1599) (end 45.3332 34.5) (width 0.2) (layer "F.Cu") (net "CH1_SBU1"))
 (segment (start 42.45 34.5) (end 42.45 33.8983) (width 0.2) (layer "F.Cu") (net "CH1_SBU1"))
 (segment (start 39.0517 33.8983) (end 39.0517 34.5) (width 0.2) (layer "F.Cu") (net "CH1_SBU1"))
 (segment (start 38.1992 33.0458) (end 33.0458 33.0458) (width 0.2) (layer "F.Cu") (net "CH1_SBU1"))
 (segment (start 38.45 34.5) (end 39.0517 34.5) (width 0.2) (layer "F.Cu") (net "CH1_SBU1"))
 (segment (start 45.9931 37.2071) (end 45.9931 35.1599) (width 0.2) (layer "F.Cu") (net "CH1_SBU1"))
 (segment (start 46.45 37.664) (end 45.9931 37.2071) (width 0.2) (layer "F.Cu") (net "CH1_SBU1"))
 (segment (start 39.0517 33.8983) (end 38.1992 33.0458) (width 0.2) (layer "F.Cu") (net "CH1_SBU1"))
 (segment (start 45.3332 34.5) (end 42.45 34.5) (width 0.2) (layer "F.Cu") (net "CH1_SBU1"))
 (segment (start 47.8803 40.068) (end 48.9483 39) (width 0.2) (layer "F.Cu") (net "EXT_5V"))
 (segment (start 33.81 31.27) (end 32.54 30) (width 0.2) (layer "F.Cu") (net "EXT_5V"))
 (segment (start 33.55 39) (end 33.55 39.6017) (width 0.2) (layer "F.Cu") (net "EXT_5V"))
 (segment (start 41.4663 40.068) (end 47.8803 40.068) (width 0.2) (layer "F.Cu") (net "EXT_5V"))
 (segment (start 27.46 30) (end 26.19 28.73) (width 0.2) (layer "F.Cu") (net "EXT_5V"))
 (segment (start 40.3983 39) (end 39.7966 39.6017) (width 0.2) (layer "F.Cu") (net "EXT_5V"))
 (segment (start 37.55 39) (end 37.55 39.6017) (width 0.2) (layer "F.Cu") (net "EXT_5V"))
 (segment (start 33.55 39.6017) (end 37.55 39.6017) (width 0.2) (layer "F.Cu") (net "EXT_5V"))
 (segment (start 39.7966 39.6017) (end 37.55 39.6017) (width 0.2) (layer "F.Cu") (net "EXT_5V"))
 (segment (start 40.3983 39) (end 41.4663 40.068) (width 0.2) (layer "F.Cu") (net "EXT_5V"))
 (segment (start 49.55 39) (end 48.9483 39) (width 0.2) (layer "F.Cu") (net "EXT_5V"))
 (segment (start 32.54 30) (end 27.46 30) (width 0.2) (layer "F.Cu") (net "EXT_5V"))
 (segment (start 41.1 39) (end 40.3983 39) (width 0.2) (layer "F.Cu") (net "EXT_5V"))
 (segment (start 36.9483 34.5) (end 36.724 34.5) (width 0.2) (layer "F.Cu") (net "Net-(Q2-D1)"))
 (segment (start 37.05 28.6999) (end 37.05 27.7982) (width 0.2) (layer "F.Cu") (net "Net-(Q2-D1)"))
 (segment (start 37.05 27.7982) (end 36.3458 27.7982) (width 0.2) (layer "F.Cu") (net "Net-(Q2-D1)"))
 (segment (start 37.55 34.5) (end 36.9483 34.5) (width 0.2) (layer "F.Cu") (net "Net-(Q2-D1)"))
 (via (at 36.724 34.5) (size 0.6) (drill 0.3) (layers "F.Cu" "B.Cu") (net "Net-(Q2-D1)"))
 (via (at 36.3458 27.7982) (size 0.6) (drill 0.3) (layers "F.Cu" "B.Cu") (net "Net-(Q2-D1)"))
 (segment (start 36.724 28.1764) (end 36.3458 27.7982) (width 0.2) (layer "B.Cu") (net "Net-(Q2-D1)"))
 (segment (start 36.724 34.5) (end 36.724 28.1764) (width 0.2) (layer "B.Cu") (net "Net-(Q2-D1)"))
 (segment (start 45.5797 37.6446) (end 36.4071 37.6446) (width 0.2) (layer "F.Cu") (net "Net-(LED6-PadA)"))
 (segment (start 50 35.55) (end 48.8147 35.55) (width 0.2) (layer "F.Cu") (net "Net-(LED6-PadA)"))
 (segment (start 36.4071 37.6446) (end 35.0517 39) (width 0.2) (layer "F.Cu") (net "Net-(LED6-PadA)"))
 (segment (start 34.45 39) (end 35.0517 39) (width 0.2) (layer "F.Cu") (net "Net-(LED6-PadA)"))
 (via (at 48.8147 35.55) (size 0.6) (drill 0.3) (layers "F.Cu" "B.Cu") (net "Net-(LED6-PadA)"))
 (via (at 45.5797 37.6446) (size 0.6) (drill 0.3) (layers "F.Cu" "B.Cu") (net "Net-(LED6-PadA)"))
 (segment (start 47.2727 37.6446) (end 45.5797 37.6446) (width 0.2) (layer "B.Cu") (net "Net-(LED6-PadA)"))
 (segment (start 48.8147 35.55) (end 48.8147 36.1026) (width 0.2) (layer "B.Cu") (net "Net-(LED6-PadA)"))
 (segment (start 48.8147 36.1026) (end 47.2727 37.6446) (width 0.2) (layer "B.Cu") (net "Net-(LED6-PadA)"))
 (segment (start 34.45 33.8998) (end 34.45 33.8983) (width 0.2) (layer "F.Cu") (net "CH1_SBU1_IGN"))
 (segment (start 31.3583 33.8983) (end 34.45 33.8983) (width 0.2) (layer "F.Cu") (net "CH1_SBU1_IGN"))
 (segment (start 34.5446 33.8037) (end 34.45 33.8983) (width 0.2) (layer "F.Cu") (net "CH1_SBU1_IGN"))
 (segment (start 34.45 34.5) (end 34.45 33.9991) (width 0.2) (layer "F.Cu") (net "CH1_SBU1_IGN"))
 (segment (start 37.05 31.3001) (end 37.05 30.8492) (width 0.2) (layer "F.Cu") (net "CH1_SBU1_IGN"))
 (segment (start 37.05 30.8492) (end 37.05 30.3984) (width 0.2) (layer "F.Cu") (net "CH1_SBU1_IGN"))
 (segment (start 34.45 33.9991) (end 34.45 33.8998) (width 0.2) (layer "F.Cu") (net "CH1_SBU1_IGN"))
 (segment (start 40.9483 30) (end 40.945 29.9967) (width 0.2) (layer "F.Cu") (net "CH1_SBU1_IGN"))
 (segment (start 41.55 30) (end 40.9483 30) (width 0.2) (layer "F.Cu") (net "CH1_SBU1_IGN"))
 (segment (start 28.73 31.27) (end 31.3583 33.8983) (width 0.2) (layer "F.Cu") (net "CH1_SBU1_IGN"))
 (segment (start 40.945 29.9967) (end 37.4517 29.9967) (width 0.2) (layer "F.Cu") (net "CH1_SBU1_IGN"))
 (segment (start 37.4517 29.9967) (end 37.05 30.3984) (width 0.2) (layer "F.Cu") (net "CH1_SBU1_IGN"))
 (segment (start 35.5614 33.8037) (end 34.5446 33.8037) (width 0.2) (layer "F.Cu") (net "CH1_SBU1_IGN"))
 (segment (start 37.05 30.8492) (end 36.1098 30.8492) (width 0.2) (layer "F.Cu") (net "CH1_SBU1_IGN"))
 (via (at 36.1098 30.8492) (size 0.6) (drill 0.3) (layers "F.Cu" "B.Cu") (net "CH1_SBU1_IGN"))
 (via (at 35.5614 33.8037) (size 0.6) (drill 0.3) (layers "F.Cu" "B.Cu") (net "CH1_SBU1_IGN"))
 (segment (start 35.5614 33.8037) (end 35.5614 31.3976) (width 0.2) (layer "B.Cu") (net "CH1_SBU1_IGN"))
 (segment (start 35.5614 31.3976) (end 36.1098 30.8492) (width 0.2) (layer "B.Cu") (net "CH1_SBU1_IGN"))
 (segment (start 44.9483 39) (end 44.9316 38.9833) (width 0.2) (layer "F.Cu") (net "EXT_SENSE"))
 (segment (start 44.9316 38.9833) (end 43.8262 38.9833) (width 0.2) (layer "F.Cu") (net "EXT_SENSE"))
 (segment (start 45.55 39) (end 44.9483 39) (width 0.2) (layer "F.Cu") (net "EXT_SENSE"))
 (via (at 43.8262 38.9833) (size 0.6) (drill 0.3) (layers "F.Cu" "B.Cu") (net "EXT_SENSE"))
 (segment (start 32.54 31.7593) (end 39.764 38.9833) (width 0.2) (layer "B.Cu") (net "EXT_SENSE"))
 (segment (start 31.27 28.73) (end 32.54 30) (width 0.2) (layer "B.Cu") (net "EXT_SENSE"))
 (segment (start 39.764 38.9833) (end 43.8262 38.9833) (width 0.2) (layer "B.Cu") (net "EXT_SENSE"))
 (segment (start 32.54 30) (end 32.54 31.7593) (width 0.2) (layer "B.Cu") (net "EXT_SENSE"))
 (segment (start 33.9483 35.5) (end 33.55 35.1017) (width 0.2) (layer "F.Cu") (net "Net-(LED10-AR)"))
 (segment (start 45.05 35.5) (end 33.9483 35.5) (width 0.2) (layer "F.Cu") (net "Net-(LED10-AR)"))
 (segment (start 33.55 34.5) (end 33.55 35.1017) (width 0.2) (layer "F.Cu") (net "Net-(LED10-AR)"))
 (segment (start 49.55 30.8486) (end 49.55 30) (width 0.2) (layer "F.Cu") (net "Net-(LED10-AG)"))
 (segment (start 47.6517 36.2017) (end 47.7323 36.2823) (width 0.2) (layer "F.Cu") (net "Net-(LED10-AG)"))
 (segment (start 46.95 35.5) (end 47.6517 35.5) (width 0.2) (layer "F.Cu") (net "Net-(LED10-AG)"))
 (segment (start 47.6517 35.5) (end 47.6517 36.2017) (width 0.2) (layer "F.Cu") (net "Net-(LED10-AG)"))
 (via (at 49.55 30.8486) (size 0.6) (drill 0.3) (layers "F.Cu" "B.Cu") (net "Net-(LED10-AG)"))
 (via (at 47.7323 36.2823) (size 0.6) (drill 0.3) (layers "F.Cu" "B.Cu") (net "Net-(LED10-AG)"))
 (segment (start 49.55 30.8486) (end 47.7323 32.6663) (width 0.2) (layer "B.Cu") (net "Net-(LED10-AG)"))
 (segment (start 47.7323 32.6663) (end 47.7323 36.2823) (width 0.2) (layer "B.Cu") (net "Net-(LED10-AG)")))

